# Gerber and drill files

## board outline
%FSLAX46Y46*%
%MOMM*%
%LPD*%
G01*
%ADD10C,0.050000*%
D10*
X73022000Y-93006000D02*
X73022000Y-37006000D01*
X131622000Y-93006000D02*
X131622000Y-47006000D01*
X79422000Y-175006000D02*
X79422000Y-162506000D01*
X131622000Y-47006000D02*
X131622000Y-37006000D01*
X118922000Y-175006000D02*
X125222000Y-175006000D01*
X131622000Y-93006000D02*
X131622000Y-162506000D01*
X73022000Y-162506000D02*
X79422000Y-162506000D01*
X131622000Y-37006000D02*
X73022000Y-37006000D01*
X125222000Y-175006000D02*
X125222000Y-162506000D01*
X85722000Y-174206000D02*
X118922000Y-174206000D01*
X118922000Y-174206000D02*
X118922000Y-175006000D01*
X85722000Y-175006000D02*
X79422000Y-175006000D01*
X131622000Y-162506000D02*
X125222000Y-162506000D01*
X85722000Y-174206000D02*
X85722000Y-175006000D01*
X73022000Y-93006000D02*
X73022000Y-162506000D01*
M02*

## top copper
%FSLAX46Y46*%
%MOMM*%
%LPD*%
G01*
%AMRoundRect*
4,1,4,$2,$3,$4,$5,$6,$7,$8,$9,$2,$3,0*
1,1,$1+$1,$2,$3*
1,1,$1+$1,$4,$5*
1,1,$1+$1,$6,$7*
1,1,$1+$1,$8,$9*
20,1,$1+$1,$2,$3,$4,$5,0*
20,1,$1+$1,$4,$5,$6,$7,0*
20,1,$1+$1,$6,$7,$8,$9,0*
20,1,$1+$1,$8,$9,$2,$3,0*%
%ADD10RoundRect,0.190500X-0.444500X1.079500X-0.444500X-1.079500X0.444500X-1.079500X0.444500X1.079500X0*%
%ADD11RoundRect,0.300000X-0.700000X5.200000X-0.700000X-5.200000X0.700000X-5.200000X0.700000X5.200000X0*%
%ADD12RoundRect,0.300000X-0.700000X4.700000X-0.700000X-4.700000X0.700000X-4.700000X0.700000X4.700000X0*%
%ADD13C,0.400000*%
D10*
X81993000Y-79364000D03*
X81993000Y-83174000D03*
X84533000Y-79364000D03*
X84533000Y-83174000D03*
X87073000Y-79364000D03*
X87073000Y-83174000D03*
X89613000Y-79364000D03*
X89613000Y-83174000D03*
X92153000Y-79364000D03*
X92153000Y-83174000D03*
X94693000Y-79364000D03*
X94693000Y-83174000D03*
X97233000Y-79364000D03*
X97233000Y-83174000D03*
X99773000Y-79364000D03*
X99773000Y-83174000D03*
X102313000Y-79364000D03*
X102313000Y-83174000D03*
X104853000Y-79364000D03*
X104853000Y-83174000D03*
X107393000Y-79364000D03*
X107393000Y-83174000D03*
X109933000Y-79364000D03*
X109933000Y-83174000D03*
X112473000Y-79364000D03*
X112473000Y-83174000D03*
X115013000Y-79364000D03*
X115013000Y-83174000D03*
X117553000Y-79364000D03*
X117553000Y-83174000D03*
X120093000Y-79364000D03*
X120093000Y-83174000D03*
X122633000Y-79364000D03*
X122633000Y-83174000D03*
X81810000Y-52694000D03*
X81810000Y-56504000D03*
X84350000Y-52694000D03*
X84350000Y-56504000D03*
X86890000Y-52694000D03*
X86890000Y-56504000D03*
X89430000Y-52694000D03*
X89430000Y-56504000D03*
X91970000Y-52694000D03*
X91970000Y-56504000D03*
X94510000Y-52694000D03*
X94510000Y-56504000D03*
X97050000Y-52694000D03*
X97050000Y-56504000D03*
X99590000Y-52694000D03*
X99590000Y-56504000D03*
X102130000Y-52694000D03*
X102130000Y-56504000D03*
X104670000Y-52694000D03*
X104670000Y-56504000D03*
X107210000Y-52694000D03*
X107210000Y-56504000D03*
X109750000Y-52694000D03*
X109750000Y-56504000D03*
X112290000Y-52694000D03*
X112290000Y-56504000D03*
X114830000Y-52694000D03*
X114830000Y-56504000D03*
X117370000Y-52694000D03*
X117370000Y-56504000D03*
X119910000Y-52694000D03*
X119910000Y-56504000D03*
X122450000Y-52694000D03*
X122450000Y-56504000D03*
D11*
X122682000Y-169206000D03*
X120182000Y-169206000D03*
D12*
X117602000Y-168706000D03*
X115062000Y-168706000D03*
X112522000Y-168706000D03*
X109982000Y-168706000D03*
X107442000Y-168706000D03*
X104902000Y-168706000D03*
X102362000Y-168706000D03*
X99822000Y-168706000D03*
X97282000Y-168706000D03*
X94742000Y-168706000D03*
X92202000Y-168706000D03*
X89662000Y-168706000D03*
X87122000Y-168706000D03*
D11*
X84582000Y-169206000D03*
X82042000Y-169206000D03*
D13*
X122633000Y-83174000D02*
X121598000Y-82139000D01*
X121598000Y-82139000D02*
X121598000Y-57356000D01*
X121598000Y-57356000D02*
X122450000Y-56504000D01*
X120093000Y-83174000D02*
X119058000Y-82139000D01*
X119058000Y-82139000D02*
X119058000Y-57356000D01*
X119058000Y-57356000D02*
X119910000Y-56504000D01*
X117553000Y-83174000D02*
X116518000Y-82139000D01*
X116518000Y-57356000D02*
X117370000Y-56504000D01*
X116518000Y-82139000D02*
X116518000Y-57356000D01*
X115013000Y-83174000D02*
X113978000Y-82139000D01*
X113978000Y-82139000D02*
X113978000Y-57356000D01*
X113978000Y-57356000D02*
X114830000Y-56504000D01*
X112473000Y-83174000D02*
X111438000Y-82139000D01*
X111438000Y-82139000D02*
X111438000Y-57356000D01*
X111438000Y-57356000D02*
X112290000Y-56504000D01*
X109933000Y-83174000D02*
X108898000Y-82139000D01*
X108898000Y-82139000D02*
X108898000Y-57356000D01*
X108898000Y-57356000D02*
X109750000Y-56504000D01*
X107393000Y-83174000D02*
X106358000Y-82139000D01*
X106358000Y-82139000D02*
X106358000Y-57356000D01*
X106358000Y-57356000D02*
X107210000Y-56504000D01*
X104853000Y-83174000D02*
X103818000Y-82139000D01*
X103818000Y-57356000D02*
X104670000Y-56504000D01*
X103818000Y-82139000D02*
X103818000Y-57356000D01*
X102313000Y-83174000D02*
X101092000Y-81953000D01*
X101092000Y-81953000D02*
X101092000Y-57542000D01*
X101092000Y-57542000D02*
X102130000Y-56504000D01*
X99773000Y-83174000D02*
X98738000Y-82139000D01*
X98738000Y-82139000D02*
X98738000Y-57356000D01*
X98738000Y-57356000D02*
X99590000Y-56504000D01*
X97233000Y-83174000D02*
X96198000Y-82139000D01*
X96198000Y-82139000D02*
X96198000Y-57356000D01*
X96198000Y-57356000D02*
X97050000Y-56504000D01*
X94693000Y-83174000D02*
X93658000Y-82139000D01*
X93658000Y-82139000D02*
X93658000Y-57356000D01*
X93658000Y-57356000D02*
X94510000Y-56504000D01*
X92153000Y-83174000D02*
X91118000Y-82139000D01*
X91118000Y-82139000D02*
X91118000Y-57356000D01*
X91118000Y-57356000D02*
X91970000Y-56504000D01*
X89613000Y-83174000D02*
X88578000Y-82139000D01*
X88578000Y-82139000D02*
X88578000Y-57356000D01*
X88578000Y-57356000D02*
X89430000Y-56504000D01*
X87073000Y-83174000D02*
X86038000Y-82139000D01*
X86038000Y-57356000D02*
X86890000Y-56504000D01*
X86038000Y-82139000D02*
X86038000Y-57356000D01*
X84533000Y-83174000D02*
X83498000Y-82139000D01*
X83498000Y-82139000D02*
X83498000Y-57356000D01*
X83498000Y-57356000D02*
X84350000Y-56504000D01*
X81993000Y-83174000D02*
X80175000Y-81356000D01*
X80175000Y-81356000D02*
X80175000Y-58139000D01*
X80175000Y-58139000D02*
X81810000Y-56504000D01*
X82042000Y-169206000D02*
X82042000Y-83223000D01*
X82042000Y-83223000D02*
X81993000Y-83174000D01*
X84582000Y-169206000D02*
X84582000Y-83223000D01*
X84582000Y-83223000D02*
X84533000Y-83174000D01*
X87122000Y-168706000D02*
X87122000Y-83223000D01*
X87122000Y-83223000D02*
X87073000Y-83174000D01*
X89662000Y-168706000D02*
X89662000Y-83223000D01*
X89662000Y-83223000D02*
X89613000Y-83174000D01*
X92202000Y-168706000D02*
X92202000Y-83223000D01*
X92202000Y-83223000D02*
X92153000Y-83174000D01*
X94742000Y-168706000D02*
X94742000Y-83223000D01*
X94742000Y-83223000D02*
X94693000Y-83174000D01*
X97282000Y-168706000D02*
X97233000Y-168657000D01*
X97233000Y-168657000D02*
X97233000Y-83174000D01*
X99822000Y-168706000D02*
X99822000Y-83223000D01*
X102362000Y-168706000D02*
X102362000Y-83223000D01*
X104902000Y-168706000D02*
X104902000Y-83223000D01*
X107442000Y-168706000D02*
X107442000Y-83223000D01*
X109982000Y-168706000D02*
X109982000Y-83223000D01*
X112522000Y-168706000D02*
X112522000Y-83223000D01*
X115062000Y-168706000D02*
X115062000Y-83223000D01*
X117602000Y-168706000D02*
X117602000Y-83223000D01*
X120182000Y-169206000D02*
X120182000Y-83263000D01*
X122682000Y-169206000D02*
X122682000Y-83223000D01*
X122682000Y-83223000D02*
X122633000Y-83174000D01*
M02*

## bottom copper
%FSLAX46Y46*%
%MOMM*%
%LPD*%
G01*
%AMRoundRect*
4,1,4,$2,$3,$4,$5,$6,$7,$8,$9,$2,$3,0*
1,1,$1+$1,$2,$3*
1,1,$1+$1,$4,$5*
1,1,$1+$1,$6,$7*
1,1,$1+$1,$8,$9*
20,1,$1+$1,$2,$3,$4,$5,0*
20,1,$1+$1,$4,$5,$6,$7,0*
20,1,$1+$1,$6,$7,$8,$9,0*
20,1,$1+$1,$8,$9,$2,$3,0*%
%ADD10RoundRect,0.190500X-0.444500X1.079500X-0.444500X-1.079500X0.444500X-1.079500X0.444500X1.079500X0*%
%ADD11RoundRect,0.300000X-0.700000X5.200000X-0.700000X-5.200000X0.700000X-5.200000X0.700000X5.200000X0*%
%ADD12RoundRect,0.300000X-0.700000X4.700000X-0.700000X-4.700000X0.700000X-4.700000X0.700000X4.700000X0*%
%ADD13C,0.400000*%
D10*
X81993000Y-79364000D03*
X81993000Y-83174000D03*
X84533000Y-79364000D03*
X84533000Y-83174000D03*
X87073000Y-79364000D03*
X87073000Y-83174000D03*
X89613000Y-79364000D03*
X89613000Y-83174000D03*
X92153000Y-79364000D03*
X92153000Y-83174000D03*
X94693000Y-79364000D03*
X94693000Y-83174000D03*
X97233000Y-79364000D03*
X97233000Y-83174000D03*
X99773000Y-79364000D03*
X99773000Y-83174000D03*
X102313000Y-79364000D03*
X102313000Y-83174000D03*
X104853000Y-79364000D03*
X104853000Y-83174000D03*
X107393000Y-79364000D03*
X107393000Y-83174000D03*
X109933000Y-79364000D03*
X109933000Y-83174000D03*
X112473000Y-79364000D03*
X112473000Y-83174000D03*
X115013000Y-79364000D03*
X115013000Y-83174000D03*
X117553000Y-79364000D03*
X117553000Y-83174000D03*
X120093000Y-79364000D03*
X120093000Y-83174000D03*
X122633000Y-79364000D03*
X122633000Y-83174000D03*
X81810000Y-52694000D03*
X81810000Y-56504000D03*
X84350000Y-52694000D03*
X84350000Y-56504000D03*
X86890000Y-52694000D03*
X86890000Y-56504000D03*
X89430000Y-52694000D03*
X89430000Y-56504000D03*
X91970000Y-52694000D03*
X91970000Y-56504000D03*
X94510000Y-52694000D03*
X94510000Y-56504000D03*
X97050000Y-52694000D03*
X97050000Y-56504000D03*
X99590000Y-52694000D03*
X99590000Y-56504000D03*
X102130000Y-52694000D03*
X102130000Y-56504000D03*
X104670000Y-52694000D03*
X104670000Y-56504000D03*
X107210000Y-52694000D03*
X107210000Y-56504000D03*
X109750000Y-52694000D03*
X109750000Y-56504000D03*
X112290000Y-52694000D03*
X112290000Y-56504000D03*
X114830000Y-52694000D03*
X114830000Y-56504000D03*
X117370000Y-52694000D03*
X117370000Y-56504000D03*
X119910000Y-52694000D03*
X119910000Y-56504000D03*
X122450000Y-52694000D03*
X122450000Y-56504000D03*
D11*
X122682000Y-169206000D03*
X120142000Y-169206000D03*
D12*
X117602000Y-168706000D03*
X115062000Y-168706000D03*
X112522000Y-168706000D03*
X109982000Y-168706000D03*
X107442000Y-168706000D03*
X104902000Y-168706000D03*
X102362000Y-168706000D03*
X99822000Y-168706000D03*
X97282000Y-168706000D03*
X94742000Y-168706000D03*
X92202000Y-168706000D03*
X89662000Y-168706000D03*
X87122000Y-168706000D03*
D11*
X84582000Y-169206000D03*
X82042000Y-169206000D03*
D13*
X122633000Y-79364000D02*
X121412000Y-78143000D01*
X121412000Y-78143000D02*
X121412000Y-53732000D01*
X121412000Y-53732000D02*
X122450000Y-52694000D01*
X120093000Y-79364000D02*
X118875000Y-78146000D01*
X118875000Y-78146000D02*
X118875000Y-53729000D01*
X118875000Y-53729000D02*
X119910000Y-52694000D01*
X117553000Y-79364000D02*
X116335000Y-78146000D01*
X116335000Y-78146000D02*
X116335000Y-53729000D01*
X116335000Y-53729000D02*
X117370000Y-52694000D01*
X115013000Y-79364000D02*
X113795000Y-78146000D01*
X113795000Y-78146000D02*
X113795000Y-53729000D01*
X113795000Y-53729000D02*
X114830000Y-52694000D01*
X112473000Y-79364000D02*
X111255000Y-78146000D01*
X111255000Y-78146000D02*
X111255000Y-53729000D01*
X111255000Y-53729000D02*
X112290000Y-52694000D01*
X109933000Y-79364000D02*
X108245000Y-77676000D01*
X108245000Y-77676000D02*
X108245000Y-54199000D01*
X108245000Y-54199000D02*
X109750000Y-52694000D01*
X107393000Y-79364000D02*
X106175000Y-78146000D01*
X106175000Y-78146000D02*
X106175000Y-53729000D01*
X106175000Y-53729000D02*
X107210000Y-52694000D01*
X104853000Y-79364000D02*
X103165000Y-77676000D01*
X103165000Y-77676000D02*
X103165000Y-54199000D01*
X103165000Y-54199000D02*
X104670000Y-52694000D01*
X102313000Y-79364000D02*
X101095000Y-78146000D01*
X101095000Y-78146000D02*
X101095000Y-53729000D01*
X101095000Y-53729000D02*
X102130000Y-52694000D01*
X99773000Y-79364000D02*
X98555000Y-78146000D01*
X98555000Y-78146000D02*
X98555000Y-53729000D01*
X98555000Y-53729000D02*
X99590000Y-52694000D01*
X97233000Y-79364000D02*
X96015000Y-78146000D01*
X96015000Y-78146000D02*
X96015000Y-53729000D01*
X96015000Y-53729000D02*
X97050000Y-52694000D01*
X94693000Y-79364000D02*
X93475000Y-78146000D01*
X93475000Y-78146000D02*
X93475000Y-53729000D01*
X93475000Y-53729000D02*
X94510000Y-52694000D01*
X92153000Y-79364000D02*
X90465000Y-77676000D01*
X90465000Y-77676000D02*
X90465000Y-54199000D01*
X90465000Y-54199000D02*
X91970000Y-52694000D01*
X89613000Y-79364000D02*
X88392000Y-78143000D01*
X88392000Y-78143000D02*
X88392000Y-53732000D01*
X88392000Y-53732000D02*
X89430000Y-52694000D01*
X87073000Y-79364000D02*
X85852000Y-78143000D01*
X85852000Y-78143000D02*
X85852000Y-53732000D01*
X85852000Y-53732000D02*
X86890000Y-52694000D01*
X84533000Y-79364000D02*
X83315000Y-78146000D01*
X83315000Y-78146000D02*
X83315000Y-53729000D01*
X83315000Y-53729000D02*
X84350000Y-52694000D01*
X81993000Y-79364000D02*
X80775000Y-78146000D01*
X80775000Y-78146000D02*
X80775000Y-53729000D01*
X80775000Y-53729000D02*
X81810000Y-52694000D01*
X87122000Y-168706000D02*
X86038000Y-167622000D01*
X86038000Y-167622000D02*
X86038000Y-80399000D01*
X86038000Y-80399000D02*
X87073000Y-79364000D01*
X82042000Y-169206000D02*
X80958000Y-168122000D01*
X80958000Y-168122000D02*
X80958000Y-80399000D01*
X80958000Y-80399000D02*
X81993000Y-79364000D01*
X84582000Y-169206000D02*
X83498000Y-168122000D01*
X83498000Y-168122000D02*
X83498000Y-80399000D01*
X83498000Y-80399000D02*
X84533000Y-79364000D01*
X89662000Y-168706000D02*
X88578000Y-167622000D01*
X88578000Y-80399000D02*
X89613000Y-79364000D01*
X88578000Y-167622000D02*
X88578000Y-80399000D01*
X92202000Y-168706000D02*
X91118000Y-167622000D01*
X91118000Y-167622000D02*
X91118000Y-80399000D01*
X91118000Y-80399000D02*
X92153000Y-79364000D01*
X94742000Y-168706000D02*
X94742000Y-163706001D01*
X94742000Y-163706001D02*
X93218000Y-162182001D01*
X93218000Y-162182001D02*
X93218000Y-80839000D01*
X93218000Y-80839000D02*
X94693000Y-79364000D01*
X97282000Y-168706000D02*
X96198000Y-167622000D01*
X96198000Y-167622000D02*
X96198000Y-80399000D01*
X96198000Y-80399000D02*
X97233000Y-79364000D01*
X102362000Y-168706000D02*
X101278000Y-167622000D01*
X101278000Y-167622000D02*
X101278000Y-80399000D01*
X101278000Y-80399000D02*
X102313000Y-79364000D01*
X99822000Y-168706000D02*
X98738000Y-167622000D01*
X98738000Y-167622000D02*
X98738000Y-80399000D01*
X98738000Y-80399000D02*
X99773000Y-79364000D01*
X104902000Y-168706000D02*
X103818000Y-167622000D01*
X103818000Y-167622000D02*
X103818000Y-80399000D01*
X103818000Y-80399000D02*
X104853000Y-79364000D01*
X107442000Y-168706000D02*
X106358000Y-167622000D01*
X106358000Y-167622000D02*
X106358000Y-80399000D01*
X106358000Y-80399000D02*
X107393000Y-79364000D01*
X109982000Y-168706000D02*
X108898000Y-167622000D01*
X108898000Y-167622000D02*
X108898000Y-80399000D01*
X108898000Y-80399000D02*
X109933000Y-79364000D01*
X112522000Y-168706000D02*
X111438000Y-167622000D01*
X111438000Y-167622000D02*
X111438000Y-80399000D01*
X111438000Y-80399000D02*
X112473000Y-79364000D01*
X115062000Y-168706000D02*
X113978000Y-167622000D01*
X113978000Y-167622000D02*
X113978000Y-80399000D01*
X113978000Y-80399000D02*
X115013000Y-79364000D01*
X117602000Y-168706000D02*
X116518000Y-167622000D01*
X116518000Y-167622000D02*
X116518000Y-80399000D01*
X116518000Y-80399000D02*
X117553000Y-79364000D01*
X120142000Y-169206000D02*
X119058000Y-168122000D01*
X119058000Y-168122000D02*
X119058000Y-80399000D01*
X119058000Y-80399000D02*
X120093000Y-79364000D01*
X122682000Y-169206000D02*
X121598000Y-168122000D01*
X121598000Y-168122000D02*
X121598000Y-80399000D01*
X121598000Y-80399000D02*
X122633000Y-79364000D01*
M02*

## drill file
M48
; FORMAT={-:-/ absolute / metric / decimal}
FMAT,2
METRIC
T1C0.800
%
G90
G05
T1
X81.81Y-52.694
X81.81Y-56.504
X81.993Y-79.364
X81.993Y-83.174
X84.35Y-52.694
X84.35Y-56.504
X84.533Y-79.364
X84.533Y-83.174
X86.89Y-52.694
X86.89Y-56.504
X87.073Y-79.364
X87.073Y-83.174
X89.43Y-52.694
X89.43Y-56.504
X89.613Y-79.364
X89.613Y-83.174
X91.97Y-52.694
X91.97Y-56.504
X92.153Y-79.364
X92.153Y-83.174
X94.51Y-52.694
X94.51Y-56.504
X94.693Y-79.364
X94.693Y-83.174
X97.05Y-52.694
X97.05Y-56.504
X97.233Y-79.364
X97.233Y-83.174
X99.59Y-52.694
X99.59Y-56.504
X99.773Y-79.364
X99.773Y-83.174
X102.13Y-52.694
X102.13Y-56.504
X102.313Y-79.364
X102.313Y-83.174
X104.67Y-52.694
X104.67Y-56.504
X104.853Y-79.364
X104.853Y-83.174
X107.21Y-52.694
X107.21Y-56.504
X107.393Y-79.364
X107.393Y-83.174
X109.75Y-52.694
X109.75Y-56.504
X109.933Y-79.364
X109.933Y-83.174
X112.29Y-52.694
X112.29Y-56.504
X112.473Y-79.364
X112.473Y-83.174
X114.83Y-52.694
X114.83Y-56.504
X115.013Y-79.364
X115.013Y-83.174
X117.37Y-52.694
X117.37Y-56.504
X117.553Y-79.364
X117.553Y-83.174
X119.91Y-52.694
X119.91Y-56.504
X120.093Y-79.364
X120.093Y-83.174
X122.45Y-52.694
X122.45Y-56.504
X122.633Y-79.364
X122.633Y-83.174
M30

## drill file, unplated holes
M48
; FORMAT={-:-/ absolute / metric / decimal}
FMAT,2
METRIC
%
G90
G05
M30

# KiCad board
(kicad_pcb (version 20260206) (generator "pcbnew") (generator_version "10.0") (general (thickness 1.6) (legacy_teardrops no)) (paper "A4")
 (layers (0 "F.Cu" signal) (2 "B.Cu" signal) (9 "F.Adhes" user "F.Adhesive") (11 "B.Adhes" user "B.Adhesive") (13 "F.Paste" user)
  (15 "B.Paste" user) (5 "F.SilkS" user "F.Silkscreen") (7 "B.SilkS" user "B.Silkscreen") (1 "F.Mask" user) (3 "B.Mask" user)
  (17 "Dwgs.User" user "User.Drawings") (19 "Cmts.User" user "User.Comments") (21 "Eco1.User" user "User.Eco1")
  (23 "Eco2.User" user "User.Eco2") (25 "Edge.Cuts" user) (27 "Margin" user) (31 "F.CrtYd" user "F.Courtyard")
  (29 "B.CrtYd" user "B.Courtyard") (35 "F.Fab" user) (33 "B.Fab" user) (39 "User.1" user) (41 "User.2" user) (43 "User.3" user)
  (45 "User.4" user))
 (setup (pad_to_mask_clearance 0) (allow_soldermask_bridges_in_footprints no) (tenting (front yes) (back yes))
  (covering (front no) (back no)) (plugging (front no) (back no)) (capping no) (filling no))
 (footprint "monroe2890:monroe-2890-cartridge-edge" (layer "F.Cu") (at 122.682 168.706 -90)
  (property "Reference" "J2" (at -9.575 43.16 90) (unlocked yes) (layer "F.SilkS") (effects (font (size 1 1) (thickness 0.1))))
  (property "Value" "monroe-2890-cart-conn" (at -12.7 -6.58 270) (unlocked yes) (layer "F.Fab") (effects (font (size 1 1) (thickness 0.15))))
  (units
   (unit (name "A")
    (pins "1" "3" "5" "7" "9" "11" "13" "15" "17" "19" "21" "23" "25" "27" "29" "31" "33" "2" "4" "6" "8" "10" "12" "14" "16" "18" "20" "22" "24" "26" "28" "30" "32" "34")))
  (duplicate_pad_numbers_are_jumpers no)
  (pad "1" smd roundrect (at 0.5 0 270) (size 11 2) (layers "F.Cu" "F.Mask" "F.Paste") (roundrect_rratio 0.15) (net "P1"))
  (pad "2" connect roundrect (at 0.5 0 270) (size 11 2) (layers "B.Cu" "B.Mask") (roundrect_rratio 0.15) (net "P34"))
  (pad "3" smd roundrect (at 0.5 2.5 270) (size 11 2) (layers "F.Cu" "F.Mask" "F.Paste") (roundrect_rratio 0.15) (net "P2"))
  (pad "4" connect roundrect (at 0.5 2.54 270) (size 11 2) (layers "B.Cu" "B.Mask") (roundrect_rratio 0.15) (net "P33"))
  (pad "5" smd roundrect (at 0 5.08 270) (size 10 2) (layers "F.Cu" "F.Mask" "F.Paste") (roundrect_rratio 0.15) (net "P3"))
  (pad "6" connect roundrect (at 0 5.08 270) (size 10 2) (layers "B.Cu" "B.Mask") (roundrect_rratio 0.15) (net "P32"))
  (pad "7" smd roundrect (at 0 7.62 270) (size 10 2) (layers "F.Cu" "F.Mask" "F.Paste") (roundrect_rratio 0.15) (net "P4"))
  (pad "8" connect roundrect (at 0 7.62 270) (size 10 2) (layers "B.Cu" "B.Mask") (roundrect_rratio 0.15) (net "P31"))
  (pad "9" smd roundrect (at 0 10.16 270) (size 10 2) (layers "F.Cu" "F.Mask" "F.Paste") (roundrect_rratio 0.15) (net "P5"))
  (pad "10" connect roundrect (at 0 10.16 270) (size 10 2) (layers "B.Cu" "B.Mask") (roundrect_rratio 0.15) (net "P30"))
  (pad "11" smd roundrect (at 0 12.7 270) (size 10 2) (layers "F.Cu" "F.Mask" "F.Paste") (roundrect_rratio 0.15) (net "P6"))
  (pad "12" connect roundrect (at 0 12.7 270) (size 10 2) (layers "B.Cu" "B.Mask") (roundrect_rratio 0.15) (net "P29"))
  (pad "13" smd roundrect (at 0 15.24 270) (size 10 2) (layers "F.Cu" "F.Mask" "F.Paste") (roundrect_rratio 0.15) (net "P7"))
  (pad "14" connect roundrect (at 0 15.24 270) (size 10 2) (layers "B.Cu" "B.Mask") (roundrect_rratio 0.15) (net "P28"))
  (pad "15" smd roundrect (at 0 17.78 270) (size 10 2) (layers "F.Cu" "F.Mask" "F.Paste") (roundrect_rratio 0.15) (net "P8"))
  (pad "16" connect roundrect (at 0 17.78 270) (size 10 2) (layers "B.Cu" "B.Mask") (roundrect_rratio 0.15) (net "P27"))
  (pad "17" smd roundrect (at 0 20.32 270) (size 10 2) (layers "F.Cu" "F.Mask" "F.Paste") (roundrect_rratio 0.15) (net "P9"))
  (pad "18" connect roundrect (at 0 20.32 270) (size 10 2) (layers "B.Cu" "B.Mask") (roundrect_rratio 0.15) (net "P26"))
  (pad "19" smd roundrect (at 0 22.86 270) (size 10 2) (layers "F.Cu" "F.Mask" "F.Paste") (roundrect_rratio 0.15) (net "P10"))
  (pad "20" connect roundrect (at 0 22.86 270) (size 10 2) (layers "B.Cu" "B.Mask") (roundrect_rratio 0.15) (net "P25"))
  (pad "21" smd roundrect (at 0 25.4 270) (size 10 2) (layers "F.Cu" "F.Mask" "F.Paste") (roundrect_rratio 0.15) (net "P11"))
  (pad "22" connect roundrect (at 0 25.4 270) (size 10 2) (layers "B.Cu" "B.Mask") (roundrect_rratio 0.15) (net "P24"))
  (pad "23" smd roundrect (at 0 27.94 270) (size 10 2) (layers "F.Cu" "F.Mask" "F.Paste") (roundrect_rratio 0.15) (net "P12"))
  (pad "24" connect roundrect (at 0 27.94 270) (size 10 2) (layers "B.Cu" "B.Mask") (roundrect_rratio 0.15) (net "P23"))
  (pad "25" smd roundrect (at 0 30.48 270) (size 10 2) (layers "F.Cu" "F.Mask" "F.Paste") (roundrect_rratio 0.15) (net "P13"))
  (pad "26" connect roundrect (at 0 30.48 270) (size 10 2) (layers "B.Cu" "B.Mask") (roundrect_rratio 0.15) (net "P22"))
  (pad "27" smd roundrect (at 0 33.02 270) (size 10 2) (layers "F.Cu" "F.Mask" "F.Paste") (roundrect_rratio 0.15) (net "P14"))
  (pad "28" connect roundrect (at 0 33.02 270) (size 10 2) (layers "B.Cu" "B.Mask") (roundrect_rratio 0.15) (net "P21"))
  (pad "29" smd roundrect (at 0 35.56 270) (size 10 2) (layers "F.Cu" "F.Mask" "F.Paste") (roundrect_rratio 0.15) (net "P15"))
  (pad "30" connect roundrect (at 0 35.56 270) (size 10 2) (layers "B.Cu" "B.Mask") (roundrect_rratio 0.15) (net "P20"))
  (pad "31" smd roundrect (at 0.5 38.1 270) (size 11 2) (layers "F.Cu" "F.Mask" "F.Paste") (roundrect_rratio 0.15) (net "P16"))
  (pad "32" connect roundrect (at 0.5 38.1 270) (size 11 2) (layers "B.Cu" "B.Mask") (roundrect_rratio 0.15) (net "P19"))
  (pad "33" smd roundrect (at 0.5 40.64 270) (size 11 2) (layers "F.Cu" "F.Mask" "F.Paste") (roundrect_rratio 0.15) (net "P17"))
  (pad "34" connect roundrect (at 0.5 40.64 270) (size 11 2) (layers "B.Cu" "B.Mask") (roundrect_rratio 0.15) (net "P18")))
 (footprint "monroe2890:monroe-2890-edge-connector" (layer "F.Cu") (at 111.457 78.856 -90)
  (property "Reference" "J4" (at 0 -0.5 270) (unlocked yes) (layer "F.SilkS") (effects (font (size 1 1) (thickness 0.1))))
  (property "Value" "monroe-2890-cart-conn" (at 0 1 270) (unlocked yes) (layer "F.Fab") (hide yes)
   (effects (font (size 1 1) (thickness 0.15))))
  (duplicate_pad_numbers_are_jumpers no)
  (pad "1" thru_hole roundrect (at 4.318 -11.176 270) (size 2.54 1.27) (drill 0.8) (layers "*.Cu" "*.Mask") (remove_unused_layers no)
   (roundrect_rratio 0.15) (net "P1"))
  (pad "2" thru_hole roundrect (at 0.508 -11.176 270) (size 2.54 1.27) (drill 0.8) (layers "*.Cu" "*.Mask") (remove_unused_layers no)
   (roundrect_rratio 0.15) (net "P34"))
  (pad "3" thru_hole roundrect (at 4.318 -8.636 270) (size 2.54 1.27) (drill 0.8) (layers "*.Cu" "*.Mask") (remove_unused_layers no)
   (roundrect_rratio 0.15) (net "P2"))
  (pad "4" thru_hole roundrect (at 0.508 -8.636 270) (size 2.54 1.27) (drill 0.8) (layers "*.Cu" "*.Mask") (remove_unused_layers no)
   (roundrect_rratio 0.15) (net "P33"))
  (pad "5" thru_hole roundrect (at 4.318 -6.096 270) (size 2.54 1.27) (drill 0.8) (layers "*.Cu" "*.Mask") (remove_unused_layers no)
   (roundrect_rratio 0.15) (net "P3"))
  (pad "6" thru_hole roundrect (at 0.508 -6.096 270) (size 2.54 1.27) (drill 0.8) (layers "*.Cu" "*.Mask") (remove_unused_layers no)
   (roundrect_rratio 0.15) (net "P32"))
  (pad "7" thru_hole roundrect (at 4.318 -3.556 270) (size 2.54 1.27) (drill 0.8) (layers "*.Cu" "*.Mask") (remove_unused_layers no)
   (roundrect_rratio 0.15) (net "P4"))
  (pad "8" thru_hole roundrect (at 0.508 -3.556 270) (size 2.54 1.27) (drill 0.8) (layers "*.Cu" "*.Mask") (remove_unused_layers no)
   (roundrect_rratio 0.15) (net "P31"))
  (pad "9" thru_hole roundrect (at 4.318 -1.016 270) (size 2.54 1.27) (drill 0.8) (layers "*.Cu" "*.Mask") (remove_unused_layers no)
   (roundrect_rratio 0.15) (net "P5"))
  (pad "10" thru_hole roundrect (at 0.508 -1.016 270) (size 2.54 1.27) (drill 0.8) (layers "*.Cu" "*.Mask") (remove_unused_layers no)
   (roundrect_rratio 0.15) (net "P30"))
  (pad "11" thru_hole roundrect (at 4.318 1.524 270) (size 2.54 1.27) (drill 0.8) (layers "*.Cu" "*.Mask") (remove_unused_layers no)
   (roundrect_rratio 0.15) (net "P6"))
  (pad "12" thru_hole roundrect (at 0.508 1.524 270) (size 2.54 1.27) (drill 0.8) (layers "*.Cu" "*.Mask") (remove_unused_layers no)
   (roundrect_rratio 0.15) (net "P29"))
  (pad "13" thru_hole roundrect (at 4.318 4.064 270) (size 2.54 1.27) (drill 0.8) (layers "*.Cu" "*.Mask") (remove_unused_layers no)
   (roundrect_rratio 0.15) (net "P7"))
  (pad "14" thru_hole roundrect (at 0.508 4.064 270) (size 2.54 1.27) (drill 0.8) (layers "*.Cu" "*.Mask") (remove_unused_layers no)
   (roundrect_rratio 0.15) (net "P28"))
  (pad "15" thru_hole roundrect (at 4.318 6.604 270) (size 2.54 1.27) (drill 0.8) (layers "*.Cu" "*.Mask") (remove_unused_layers no)
   (roundrect_rratio 0.15) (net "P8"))
  (pad "16" thru_hole roundrect (at 0.508 6.604 270) (size 2.54 1.27) (drill 0.8) (layers "*.Cu" "*.Mask") (remove_unused_layers no)
   (roundrect_rratio 0.15) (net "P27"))
  (pad "17" thru_hole roundrect (at 4.318 9.144 270) (size 2.54 1.27) (drill 0.8) (layers "*.Cu" "*.Mask") (remove_unused_layers no)
   (roundrect_rratio 0.15) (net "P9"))
  (pad "18" thru_hole roundrect (at 0.508 9.144 270) (size 2.54 1.27) (drill 0.8) (layers "*.Cu" "*.Mask") (remove_unused_layers no)
   (roundrect_rratio 0.15) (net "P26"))
  (pad "19" thru_hole roundrect (at 4.318 11.684 270) (size 2.54 1.27) (drill 0.8) (layers "*.Cu" "*.Mask") (remove_unused_layers no)
   (roundrect_rratio 0.15) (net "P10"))
  (pad "20" thru_hole roundrect (at 0.508 11.684 270) (size 2.54 1.27) (drill 0.8) (layers "*.Cu" "*.Mask") (remove_unused_layers no)
   (roundrect_rratio 0.15) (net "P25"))
  (pad "21" thru_hole roundrect (at 4.318 14.224 270) (size 2.54 1.27) (drill 0.8) (layers "*.Cu" "*.Mask") (remove_unused_layers no)
   (roundrect_rratio 0.15) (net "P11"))
  (pad "22" thru_hole roundrect (at 0.508 14.224 270) (size 2.54 1.27) (drill 0.8) (layers "*.Cu" "*.Mask") (remove_unused_layers no)
   (roundrect_rratio 0.15) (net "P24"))
  (pad "23" thru_hole roundrect (at 4.318 16.764 270) (size 2.54 1.27) (drill 0.8) (layers "*.Cu" "*.Mask") (remove_unused_layers no)
   (roundrect_rratio 0.15) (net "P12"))
  (pad "24" thru_hole roundrect (at 0.508 16.764 270) (size 2.54 1.27) (drill 0.8) (layers "*.Cu" "*.Mask") (remove_unused_layers no)
   (roundrect_rratio 0.15) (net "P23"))
  (pad "25" thru_hole roundrect (at 4.318 19.304 270) (size 2.54 1.27) (drill 0.8) (layers "*.Cu" "*.Mask") (remove_unused_layers no)
   (roundrect_rratio 0.15) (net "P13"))
  (pad "26" thru_hole roundrect (at 0.508 19.304 270) (size 2.54 1.27) (drill 0.8) (layers "*.Cu" "*.Mask") (remove_unused_layers no)
   (roundrect_rratio 0.15) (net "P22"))
  (pad "27" thru_hole roundrect (at 4.318 21.844 270) (size 2.54 1.27) (drill 0.8) (layers "*.Cu" "*.Mask") (remove_unused_layers no)
   (roundrect_rratio 0.15) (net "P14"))
  (pad "28" thru_hole roundrect (at 0.508 21.844 270) (size 2.54 1.27) (drill 0.8) (layers "*.Cu" "*.Mask") (remove_unused_layers no)
   (roundrect_rratio 0.15) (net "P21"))
  (pad "29" thru_hole roundrect (at 4.318 24.384 270) (size 2.54 1.27) (drill 0.8) (layers "*.Cu" "*.Mask") (remove_unused_layers no)
   (roundrect_rratio 0.15) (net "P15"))
  (pad "30" thru_hole roundrect (at 0.508 24.384 270) (size 2.54 1.27) (drill 0.8) (layers "*.Cu" "*.Mask") (remove_unused_layers no)
   (roundrect_rratio 0.15) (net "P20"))
  (pad "31" thru_hole roundrect (at 4.318 26.924 270) (size 2.54 1.27) (drill 0.8) (layers "*.Cu" "*.Mask") (remove_unused_layers no)
   (roundrect_rratio 0.15) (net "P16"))
  (pad "32" thru_hole roundrect (at 0.508 26.924 270) (size 2.54 1.27) (drill 0.8) (layers "*.Cu" "*.Mask") (remove_unused_layers no)
   (roundrect_rratio 0.15) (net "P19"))
  (pad "33" thru_hole roundrect (at 4.318 29.464 270) (size 2.54 1.27) (drill 0.8) (layers "*.Cu" "*.Mask") (remove_unused_layers no)
   (roundrect_rratio 0.15) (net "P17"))
  (pad "34" thru_hole roundrect (at 0.508 29.464 270) (size 2.54 1.27) (drill 0.8) (layers "*.Cu" "*.Mask") (remove_unused_layers no)
   (roundrect_rratio 0.15) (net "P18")))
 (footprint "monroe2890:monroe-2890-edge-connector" (layer "F.Cu") (at 111.274 52.186 -90)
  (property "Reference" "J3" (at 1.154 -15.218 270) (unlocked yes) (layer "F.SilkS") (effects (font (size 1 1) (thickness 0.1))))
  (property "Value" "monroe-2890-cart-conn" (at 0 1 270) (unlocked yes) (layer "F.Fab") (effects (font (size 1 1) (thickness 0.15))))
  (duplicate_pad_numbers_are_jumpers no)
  (pad "1" thru_hole roundrect (at 4.318 -11.176 270) (size 2.54 1.27) (drill 0.8) (layers "*.Cu" "*.Mask") (remove_unused_layers no)
   (roundrect_rratio 0.15) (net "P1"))
  (pad "2" thru_hole roundrect (at 0.508 -11.176 270) (size 2.54 1.27) (drill 0.8) (layers "*.Cu" "*.Mask") (remove_unused_layers no)
   (roundrect_rratio 0.15) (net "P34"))
  (pad "3" thru_hole roundrect (at 4.318 -8.636 270) (size 2.54 1.27) (drill 0.8) (layers "*.Cu" "*.Mask") (remove_unused_layers no)
   (roundrect_rratio 0.15) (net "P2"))
  (pad "4" thru_hole roundrect (at 0.508 -8.636 270) (size 2.54 1.27) (drill 0.8) (layers "*.Cu" "*.Mask") (remove_unused_layers no)
   (roundrect_rratio 0.15) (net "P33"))
  (pad "5" thru_hole roundrect (at 4.318 -6.096 270) (size 2.54 1.27) (drill 0.8) (layers "*.Cu" "*.Mask") (remove_unused_layers no)
   (roundrect_rratio 0.15) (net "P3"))
  (pad "6" thru_hole roundrect (at 0.508 -6.096 270) (size 2.54 1.27) (drill 0.8) (layers "*.Cu" "*.Mask") (remove_unused_layers no)
   (roundrect_rratio 0.15) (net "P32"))
  (pad "7" thru_hole roundrect (at 4.318 -3.556 270) (size 2.54 1.27) (drill 0.8) (layers "*.Cu" "*.Mask") (remove_unused_layers no)
   (roundrect_rratio 0.15) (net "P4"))
  (pad "8" thru_hole roundrect (at 0.508 -3.556 270) (size 2.54 1.27) (drill 0.8) (layers "*.Cu" "*.Mask") (remove_unused_layers no)
   (roundrect_rratio 0.15) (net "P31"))
  (pad "9" thru_hole roundrect (at 4.318 -1.016 270) (size 2.54 1.27) (drill 0.8) (layers "*.Cu" "*.Mask") (remove_unused_layers no)
   (roundrect_rratio 0.15) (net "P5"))
  (pad "10" thru_hole roundrect (at 0.508 -1.016 270) (size 2.54 1.27) (drill 0.8) (layers "*.Cu" "*.Mask") (remove_unused_layers no)
   (roundrect_rratio 0.15) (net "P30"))
  (pad "11" thru_hole roundrect (at 4.318 1.524 270) (size 2.54 1.27) (drill 0.8) (layers "*.Cu" "*.Mask") (remove_unused_layers no)
   (roundrect_rratio 0.15) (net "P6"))
  (pad "12" thru_hole roundrect (at 0.508 1.524 270) (size 2.54 1.27) (drill 0.8) (layers "*.Cu" "*.Mask") (remove_unused_layers no)
   (roundrect_rratio 0.15) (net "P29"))
  (pad "13" thru_hole roundrect (at 4.318 4.064 270) (size 2.54 1.27) (drill 0.8) (layers "*.Cu" "*.Mask") (remove_unused_layers no)
   (roundrect_rratio 0.15) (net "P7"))
  (pad "14" thru_hole roundrect (at 0.508 4.064 270) (size 2.54 1.27) (drill 0.8) (layers "*.Cu" "*.Mask") (remove_unused_layers no)
   (roundrect_rratio 0.15) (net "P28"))
  (pad "15" thru_hole roundrect (at 4.318 6.604 270) (size 2.54 1.27) (drill 0.8) (layers "*.Cu" "*.Mask") (remove_unused_layers no)
   (roundrect_rratio 0.15) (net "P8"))
  (pad "16" thru_hole roundrect (at 0.508 6.604 270) (size 2.54 1.27) (drill 0.8) (layers "*.Cu" "*.Mask") (remove_unused_layers no)
   (roundrect_rratio 0.15) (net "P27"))
  (pad "17" thru_hole roundrect (at 4.318 9.144 270) (size 2.54 1.27) (drill 0.8) (layers "*.Cu" "*.Mask") (remove_unused_layers no)
   (roundrect_rratio 0.15) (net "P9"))
  (pad "18" thru_hole roundrect (at 0.508 9.144 270) (size 2.54 1.27) (drill 0.8) (layers "*.Cu" "*.Mask") (remove_unused_layers no)
   (roundrect_rratio 0.15) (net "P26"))
  (pad "19" thru_hole roundrect (at 4.318 11.684 270) (size 2.54 1.27) (drill 0.8) (layers "*.Cu" "*.Mask") (remove_unused_layers no)
   (roundrect_rratio 0.15) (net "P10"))
  (pad "20" thru_hole roundrect (at 0.508 11.684 270) (size 2.54 1.27) (drill 0.8) (layers "*.Cu" "*.Mask") (remove_unused_layers no)
   (roundrect_rratio 0.15) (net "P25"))
  (pad "21" thru_hole roundrect (at 4.318 14.224 270) (size 2.54 1.27) (drill 0.8) (layers "*.Cu" "*.Mask") (remove_unused_layers no)
   (roundrect_rratio 0.15) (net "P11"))
  (pad "22" thru_hole roundrect (at 0.508 14.224 270) (size 2.54 1.27) (drill 0.8) (layers "*.Cu" "*.Mask") (remove_unused_layers no)
   (roundrect_rratio 0.15) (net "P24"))
  (pad "23" thru_hole roundrect (at 4.318 16.764 270) (size 2.54 1.27) (drill 0.8) (layers "*.Cu" "*.Mask") (remove_unused_layers no)
   (roundrect_rratio 0.15) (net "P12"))
  (pad "24" thru_hole roundrect (at 0.508 16.764 270) (size 2.54 1.27) (drill 0.8) (layers "*.Cu" "*.Mask") (remove_unused_layers no)
   (roundrect_rratio 0.15) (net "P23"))
  (pad "25" thru_hole roundrect (at 4.318 19.304 270) (size 2.54 1.27) (drill 0.8) (layers "*.Cu" "*.Mask") (remove_unused_layers no)
   (roundrect_rratio 0.15) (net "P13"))
  (pad "26" thru_hole roundrect (at 0.508 19.304 270) (size 2.54 1.27) (drill 0.8) (layers "*.Cu" "*.Mask") (remove_unused_layers no)
   (roundrect_rratio 0.15) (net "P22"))
  (pad "27" thru_hole roundrect (at 4.318 21.844 270) (size 2.54 1.27) (drill 0.8) (layers "*.Cu" "*.Mask") (remove_unused_layers no)
   (roundrect_rratio 0.15) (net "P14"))
  (pad "28" thru_hole roundrect (at 0.508 21.844 270) (size 2.54 1.27) (drill 0.8) (layers "*.Cu" "*.Mask") (remove_unused_layers no)
   (roundrect_rratio 0.15) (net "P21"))
  (pad "29" thru_hole roundrect (at 4.318 24.384 270) (size 2.54 1.27) (drill 0.8) (layers "*.Cu" "*.Mask") (remove_unused_layers no)
   (roundrect_rratio 0.15) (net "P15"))
  (pad "30" thru_hole roundrect (at 0.508 24.384 270) (size 2.54 1.27) (drill 0.8) (layers "*.Cu" "*.Mask") (remove_unused_layers no)
   (roundrect_rratio 0.15) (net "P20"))
  (pad "31" thru_hole roundrect (at 4.318 26.924 270) (size 2.54 1.27) (drill 0.8) (layers "*.Cu" "*.Mask") (remove_unused_layers no)
   (roundrect_rratio 0.15) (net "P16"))
  (pad "32" thru_hole roundrect (at 0.508 26.924 270) (size 2.54 1.27) (drill 0.8) (layers "*.Cu" "*.Mask") (remove_unused_layers no)
   (roundrect_rratio 0.15) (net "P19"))
  (pad "33" thru_hole roundrect (at 4.318 29.464 270) (size 2.54 1.27) (drill 0.8) (layers "*.Cu" "*.Mask") (remove_unused_layers no)
   (roundrect_rratio 0.15) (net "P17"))
  (pad "34" thru_hole roundrect (at 0.508 29.464 270) (size 2.54 1.27) (drill 0.8) (layers "*.Cu" "*.Mask") (remove_unused_layers no)
   (roundrect_rratio 0.15) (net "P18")))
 (gr_line (start 73.022 93.006) (end 73.022 37.006) (stroke (width 0.05) (type default)) (layer "Edge.Cuts"))
 (gr_line (start 73.022 93.006) (end 73.022 162.506) (stroke (width 0.05) (type default)) (layer "Edge.Cuts"))
 (gr_line (start 73.022 162.506) (end 79.422 162.506) (stroke (width 0.05) (type default)) (layer "Edge.Cuts"))
 (gr_line (start 79.422 175.006) (end 79.422 162.506) (stroke (width 0.05) (type default)) (layer "Edge.Cuts"))
 (gr_line (start 85.722 174.206) (end 85.722 175.006) (stroke (width 0.05) (type default)) (layer "Edge.Cuts"))
 (gr_line (start 85.722 174.206) (end 118.922 174.206) (stroke (width 0.05) (type default)) (layer "Edge.Cuts"))
 (gr_line (start 85.722 175.006) (end 79.422 175.006) (stroke (width 0.05) (type default)) (layer "Edge.Cuts"))
 (gr_line (start 118.922 174.206) (end 118.922 175.006) (stroke (width 0.05) (type default)) (layer "Edge.Cuts"))
 (gr_line (start 118.922 175.006) (end 125.222 175.006) (stroke (width 0.05) (type default)) (layer "Edge.Cuts"))
 (gr_line (start 125.222 175.006) (end 125.222 162.506) (stroke (width 0.05) (type default)) (layer "Edge.Cuts"))
 (gr_line (start 131.622 37.006) (end 73.022 37.006) (stroke (width 0.05) (type default)) (layer "Edge.Cuts"))
 (gr_line (start 131.622 47.006) (end 131.622 37.006) (stroke (width 0.05) (type default)) (layer "Edge.Cuts"))
 (gr_line (start 131.622 93.006) (end 131.622 47.006) (stroke (width 0.05) (type default)) (layer "Edge.Cuts"))
 (gr_line (start 131.622 93.006) (end 131.622 162.506) (stroke (width 0.05) (type default)) (layer "Edge.Cuts"))
 (gr_line (start 131.622 162.506) (end 125.222 162.506) (stroke (width 0.05) (type default)) (layer "Edge.Cuts"))
 (segment (start 98.738 82.139) (end 98.738 57.356) (width 0.4) (layer "F.Cu") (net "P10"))
 (segment (start 99.773 83.174) (end 98.738 82.139) (width 0.4) (layer "F.Cu") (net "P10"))
 (segment (start 99.822 168.706) (end 99.822 83.223) (width 0.4) (layer "F.Cu") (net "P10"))
 (segment (start 98.738 57.356) (end 99.59 56.504) (width 0.4) (layer "F.Cu") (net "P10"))
 (segment (start 113.978 80.399) (end 115.013 79.364) (width 0.4) (layer "B.Cu") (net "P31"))
 (segment (start 113.978 167.622) (end 113.978 80.399) (width 0.4) (layer "B.Cu") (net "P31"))
 (segment (start 113.795 53.729) (end 114.83 52.694) (width 0.4) (layer "B.Cu") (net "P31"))
 (segment (start 113.795 78.146) (end 113.795 53.729) (width 0.4) (layer "B.Cu") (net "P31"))
 (segment (start 115.062 168.706) (end 113.978 167.622) (width 0.4) (layer "B.Cu") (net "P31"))
 (segment (start 115.013 79.364) (end 113.795 78.146) (width 0.4) (layer "B.Cu") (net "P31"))
 (segment (start 115.062 168.706) (end 115.062 83.223) (width 0.4) (layer "F.Cu") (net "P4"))
 (segment (start 115.013 83.174) (end 113.978 82.139) (width 0.4) (layer "F.Cu") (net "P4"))
 (segment (start 113.978 57.356) (end 114.83 56.504) (width 0.4) (layer "F.Cu") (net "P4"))
 (segment (start 113.978 82.139) (end 113.978 57.356) (width 0.4) (layer "F.Cu") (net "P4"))
 (segment (start 84.582 169.206) (end 83.498 168.122) (width 0.4) (layer "B.Cu") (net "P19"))
 (segment (start 83.315 53.729) (end 84.35 52.694) (width 0.4) (layer "B.Cu") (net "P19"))
 (segment (start 84.533 79.364) (end 83.315 78.146) (width 0.4) (layer "B.Cu") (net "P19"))
 (segment (start 83.315 78.146) (end 83.315 53.729) (width 0.4) (layer "B.Cu") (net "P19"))
 (segment (start 83.498 168.122) (end 83.498 80.399) (width 0.4) (layer "B.Cu") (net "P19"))
 (segment (start 83.498 80.399) (end 84.533 79.364) (width 0.4) (layer "B.Cu") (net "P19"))
 (segment (start 93.218 80.839) (end 94.693 79.364) (width 0.4) (layer "B.Cu") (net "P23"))
 (segment (start 93.218 162.182001) (end 93.218 80.839) (width 0.4) (layer "B.Cu") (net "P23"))
 (segment (start 94.742 163.706001) (end 93.218 162.182001) (width 0.4) (layer "B.Cu") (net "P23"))
 (segment (start 93.475 53.729) (end 94.51 52.694) (width 0.4) (layer "B.Cu") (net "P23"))
 (segment (start 94.742 168.706) (end 94.742 163.706001) (width 0.4) (layer "B.Cu") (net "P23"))
 (segment (start 93.475 78.146) (end 93.475 53.729) (width 0.4) (layer "B.Cu") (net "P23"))
 (segment (start 94.693 79.364) (end 93.475 78.146) (width 0.4) (layer "B.Cu") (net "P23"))
 (segment (start 107.393 83.174) (end 106.358 82.139) (width 0.4) (layer "F.Cu") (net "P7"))
 (segment (start 106.358 57.356) (end 107.21 56.504) (width 0.4) (layer "F.Cu") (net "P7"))
 (segment (start 107.442 168.706) (end 107.442 83.223) (width 0.4) (layer "F.Cu") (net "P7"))
 (segment (start 106.358 82.139) (end 106.358 57.356) (width 0.4) (layer "F.Cu") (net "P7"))
 (segment (start 97.233 83.174) (end 96.198 82.139) (width 0.4) (layer "F.Cu") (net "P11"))
 (segment (start 97.233 168.657) (end 97.233 83.174) (width 0.4) (layer "F.Cu") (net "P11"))
 (segment (start 96.198 57.356) (end 97.05 56.504) (width 0.4) (layer "F.Cu") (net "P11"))
 (segment (start 96.198 82.139) (end 96.198 57.356) (width 0.4) (layer "F.Cu") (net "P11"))
 (segment (start 97.282 168.706) (end 97.233 168.657) (width 0.4) (layer "F.Cu") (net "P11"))
 (segment (start 103.818 80.399) (end 104.853 79.364) (width 0.4) (layer "B.Cu") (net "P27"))
 (segment (start 104.853 79.364) (end 103.165 77.676) (width 0.4) (layer "B.Cu") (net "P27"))
 (segment (start 103.165 77.676) (end 103.165 54.199) (width 0.4) (layer "B.Cu") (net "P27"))
 (segment (start 103.818 167.622) (end 103.818 80.399) (width 0.4) (layer "B.Cu") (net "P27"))
 (segment (start 104.902 168.706) (end 103.818 167.622) (width 0.4) (layer "B.Cu") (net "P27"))
 (segment (start 103.165 54.199) (end 104.67 52.694) (width 0.4) (layer "B.Cu") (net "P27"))
 (segment (start 81.993 83.174) (end 80.175 81.356) (width 0.4) (layer "F.Cu") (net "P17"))
 (segment (start 82.042 83.223) (end 81.993 83.174) (width 0.4) (layer "F.Cu") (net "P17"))
 (segment (start 80.175 81.356) (end 80.175 58.139) (width 0.4) (layer "F.Cu") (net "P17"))
 (segment (start 80.175 58.139) (end 81.81 56.504) (width 0.4) (layer "F.Cu") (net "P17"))
 (segment (start 82.042 169.206) (end 82.042 83.223) (width 0.4) (layer "F.Cu") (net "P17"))
 (segment (start 89.613 79.364) (end 88.392 78.143) (width 0.4) (layer "B.Cu") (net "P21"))
 (segment (start 88.392 53.732) (end 89.43 52.694) (width 0.4) (layer "B.Cu") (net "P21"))
 (segment (start 88.578 80.399) (end 89.613 79.364) (width 0.4) (layer "B.Cu") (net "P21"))
 (segment (start 88.578 167.622) (end 88.578 80.399) (width 0.4) (layer "B.Cu") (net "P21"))
 (segment (start 88.392 78.143) (end 88.392 53.732) (width 0.4) (layer "B.Cu") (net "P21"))
 (segment (start 89.662 168.706) (end 88.578 167.622) (width 0.4) (layer "B.Cu") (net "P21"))
 (segment (start 111.255 53.729) (end 112.29 52.694) (width 0.4) (layer "B.Cu") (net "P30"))
 (segment (start 111.255 78.146) (end 111.255 53.729) (width 0.4) (layer "B.Cu") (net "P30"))
 (segment (start 112.473 79.364) (end 111.255 78.146) (width 0.4) (layer "B.Cu") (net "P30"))
 (segment (start 111.438 80.399) (end 112.473 79.364) (width 0.4) (layer "B.Cu") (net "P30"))
 (segment (start 112.522 168.706) (end 111.438 167.622) (width 0.4) (layer "B.Cu") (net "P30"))
 (segment (start 111.438 167.622) (end 111.438 80.399) (width 0.4) (layer "B.Cu") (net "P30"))
 (segment (start 88.578 82.139) (end 88.578 57.356) (width 0.4) (layer "F.Cu") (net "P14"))
 (segment (start 89.662 83.223) (end 89.613 83.174) (width 0.4) (layer "F.Cu") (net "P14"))
 (segment (start 88.578 57.356) (end 89.43 56.504) (width 0.4) (layer "F.Cu") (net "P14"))
 (segment (start 89.662 168.706) (end 89.662 83.223) (width 0.4) (layer "F.Cu") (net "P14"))
 (segment (start 89.613 83.174) (end 88.578 82.139) (width 0.4) (layer "F.Cu") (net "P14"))
 (segment (start 86.038 57.356) (end 86.89 56.504) (width 0.4) (layer "F.Cu") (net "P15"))
 (segment (start 87.122 83.223) (end 87.073 83.174) (width 0.4) (layer "F.Cu") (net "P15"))
 (segment (start 87.073 83.174) (end 86.038 82.139) (width 0.4) (layer "F.Cu") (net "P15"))
 (segment (start 86.038 82.139) (end 86.038 57.356) (width 0.4) (layer "F.Cu") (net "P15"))
 (segment (start 87.122 168.706) (end 87.122 83.223) (width 0.4) (layer "F.Cu") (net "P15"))
 (segment (start 120.093 79.364) (end 118.875 78.146) (width 0.4) (layer "B.Cu") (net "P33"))
 (segment (start 119.058 168.122) (end 119.058 80.399) (width 0.4) (layer "B.Cu") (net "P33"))
 (segment (start 118.875 78.146) (end 118.875 53.729) (width 0.4) (layer "B.Cu") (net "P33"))
 (segment (start 119.058 80.399) (end 120.093 79.364) (width 0.4) (layer "B.Cu") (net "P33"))
 (segment (start 120.142 169.206) (end 119.058 168.122) (width 0.4) (layer "B.Cu") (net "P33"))
 (segment (start 118.875 53.729) (end 119.91 52.694) (width 0.4) (layer "B.Cu") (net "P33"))
 (segment (start 91.118 80.399) (end 92.153 79.364) (width 0.4) (layer "B.Cu") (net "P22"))
 (segment (start 92.153 79.364) (end 90.465 77.676) (width 0.4) (layer "B.Cu") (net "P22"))
 (segment (start 90.465 77.676) (end 90.465 54.199) (width 0.4) (layer "B.Cu") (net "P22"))
 (segment (start 90.465 54.199) (end 91.97 52.694) (width 0.4) (layer "B.Cu") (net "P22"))
 (segment (start 91.118 167.622) (end 91.118 80.399) (width 0.4) (layer "B.Cu") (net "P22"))
 (segment (start 92.202 168.706) (end 91.118 167.622) (width 0.4) (layer "B.Cu") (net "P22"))
 (segment (start 107.442 168.706) (end 106.358 167.622) (width 0.4) (layer "B.Cu") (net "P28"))
 (segment (start 106.175 53.729) (end 107.21 52.694) (width 0.4) (layer "B.Cu") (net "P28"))
 (segment (start 106.175 78.146) (end 106.175 53.729) (width 0.4) (layer "B.Cu") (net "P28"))
 (segment (start 106.358 80.399) (end 107.393 79.364) (width 0.4) (layer "B.Cu") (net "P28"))
 (segment (start 107.393 79.364) (end 106.175 78.146) (width 0.4) (layer "B.Cu") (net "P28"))
 (segment (start 106.358 167.622) (end 106.358 80.399) (width 0.4) (layer "B.Cu") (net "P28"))
 (segment (start 92.202 83.223) (end 92.153 83.174) (width 0.4) (layer "F.Cu") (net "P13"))
 (segment (start 92.153 83.174) (end 91.118 82.139) (width 0.4) (layer "F.Cu") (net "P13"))
 (segment (start 92.202 168.706) (end 92.202 83.223) (width 0.4) (layer "F.Cu") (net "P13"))
 (segment (start 91.118 82.139) (end 91.118 57.356) (width 0.4) (layer "F.Cu") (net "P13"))
 (segment (start 91.118 57.356) (end 91.97 56.504) (width 0.4) (layer "F.Cu") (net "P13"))
 (segment (start 108.898 82.139) (end 108.898 57.356) (width 0.4) (layer "F.Cu") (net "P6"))
 (segment (start 108.898 57.356) (end 109.75 56.504) (width 0.4) (layer "F.Cu") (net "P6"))
 (segment (start 109.982 168.706) (end 109.982 83.223) (width 0.4) (layer "F.Cu") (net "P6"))
 (segment (start 109.933 83.174) (end 108.898 82.139) (width 0.4) (layer "F.Cu") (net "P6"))
 (segment (start 116.335 78.146) (end 116.335 53.729) (width 0.4) (layer "B.Cu") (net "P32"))
 (segment (start 116.518 167.622) (end 116.518 80.399) (width 0.4) (layer "B.Cu") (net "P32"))
 (segment (start 116.335 53.729) (end 117.37 52.694) (width 0.4) (layer "B.Cu") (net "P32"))
 (segment (start 117.602 168.706) (end 116.518 167.622) (width 0.4) (layer "B.Cu") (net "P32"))
 (segment (start 116.518 80.399) (end 117.553 79.364) (width 0.4) (layer "B.Cu") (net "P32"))
 (segment (start 117.553 79.364) (end 116.335 78.146) (width 0.4) (layer "B.Cu") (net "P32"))
 (segment (start 80.958 168.122) (end 80.958 80.399) (width 0.4) (layer "B.Cu") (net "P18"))
 (segment (start 81.993 79.364) (end 80.775 78.146) (width 0.4) (layer "B.Cu") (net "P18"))
 (segment (start 80.775 53.729) (end 81.81 52.694) (width 0.4) (layer "B.Cu") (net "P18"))
 (segment (start 80.775 78.146) (end 80.775 53.729) (width 0.4) (layer "B.Cu") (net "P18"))
 (segment (start 80.958 80.399) (end 81.993 79.364) (width 0.4) (layer "B.Cu") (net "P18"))
 (segment (start 82.042 169.206) (end 80.958 168.122) (width 0.4) (layer "B.Cu") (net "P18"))
 (segment (start 102.362 168.706) (end 102.362 83.223) (width 0.4) (layer "F.Cu") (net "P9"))
 (segment (start 101.092 57.542) (end 102.13 56.504) (width 0.4) (layer "F.Cu") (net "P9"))
 (segment (start 101.092 81.953) (end 101.092 57.542) (width 0.4) (layer "F.Cu") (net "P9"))
 (segment (start 102.313 83.174) (end 101.092 81.953) (width 0.4) (layer "F.Cu") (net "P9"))
 (segment (start 108.898 167.622) (end 108.898 80.399) (width 0.4) (layer "B.Cu") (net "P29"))
 (segment (start 109.982 168.706) (end 108.898 167.622) (width 0.4) (layer "B.Cu") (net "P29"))
 (segment (start 108.898 80.399) (end 109.933 79.364) (width 0.4) (layer "B.Cu") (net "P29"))
 (segment (start 108.245 54.199) (end 109.75 52.694) (width 0.4) (layer "B.Cu") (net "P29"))
 (segment (start 108.245 77.676) (end 108.245 54.199) (width 0.4) (layer "B.Cu") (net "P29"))
 (segment (start 109.933 79.364) (end 108.245 77.676) (width 0.4) (layer "B.Cu") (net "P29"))
 (segment (start 87.073 79.364) (end 85.852 78.143) (width 0.4) (layer "B.Cu") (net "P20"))
 (segment (start 85.852 78.143) (end 85.852 53.732) (width 0.4) (layer "B.Cu") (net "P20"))
 (segment (start 85.852 53.732) (end 86.89 52.694) (width 0.4) (layer "B.Cu") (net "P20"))
 (segment (start 87.122 168.706) (end 86.038 167.622) (width 0.4) (layer "B.Cu") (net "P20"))
 (segment (start 86.038 167.622) (end 86.038 80.399) (width 0.4) (layer "B.Cu") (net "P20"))
 (segment (start 86.038 80.399) (end 87.073 79.364) (width 0.4) (layer "B.Cu") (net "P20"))
 (segment (start 104.853 83.174) (end 103.818 82.139) (width 0.4) (layer "F.Cu") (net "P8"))
 (segment (start 103.818 57.356) (end 104.67 56.504) (width 0.4) (layer "F.Cu") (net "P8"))
 (segment (start 104.902 168.706) (end 104.902 83.223) (width 0.4) (layer "F.Cu") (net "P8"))
 (segment (start 103.818 82.139) (end 103.818 57.356) (width 0.4) (layer "F.Cu") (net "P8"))
 (segment (start 117.553 83.174) (end 116.518 82.139) (width 0.4) (layer "F.Cu") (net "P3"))
 (segment (start 116.518 57.356) (end 117.37 56.504) (width 0.4) (layer "F.Cu") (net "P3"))
 (segment (start 116.518 82.139) (end 116.518 57.356) (width 0.4) (layer "F.Cu") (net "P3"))
 (segment (start 117.602 168.706) (end 117.602 83.223) (width 0.4) (layer "F.Cu") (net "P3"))
 (segment (start 97.282 168.706) (end 96.198 167.622) (width 0.4) (layer "B.Cu") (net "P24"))
 (segment (start 96.198 80.399) (end 97.233 79.364) (width 0.4) (layer "B.Cu") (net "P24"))
 (segment (start 96.015 53.729) (end 97.05 52.694) (width 0.4) (layer "B.Cu") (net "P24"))
 (segment (start 97.233 79.364) (end 96.015 78.146) (width 0.4) (layer "B.Cu") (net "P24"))
 (segment (start 96.015 78.146) (end 96.015 53.729) (width 0.4) (layer "B.Cu") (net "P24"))
 (segment (start 96.198 167.622) (end 96.198 80.399) (width 0.4) (layer "B.Cu") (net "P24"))
 (segment (start 121.598 57.356) (end 122.45 56.504) (width 0.4) (layer "F.Cu") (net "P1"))
 (segment (start 122.682 83.223) (end 122.633 83.174) (width 0.4) (layer "F.Cu") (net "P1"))
 (segment (start 122.633 83.174) (end 121.598 82.139) (width 0.4) (layer "F.Cu") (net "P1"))
 (segment (start 122.682 169.206) (end 122.682 83.223) (width 0.4) (layer "F.Cu") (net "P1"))
 (segment (start 121.598 82.139) (end 121.598 57.356) (width 0.4) (layer "F.Cu") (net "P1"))
 (segment (start 121.598 80.399) (end 122.633 79.364) (width 0.4) (layer "B.Cu") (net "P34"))
 (segment (start 122.633 79.364) (end 121.412 78.143) (width 0.4) (layer "B.Cu") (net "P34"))
 (segment (start 122.682 169.206) (end 121.598 168.122) (width 0.4) (layer "B.Cu") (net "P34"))
 (segment (start 121.412 53.732) (end 122.45 52.694) (width 0.4) (layer "B.Cu") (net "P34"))
 (segment (start 121.598 168.122) (end 121.598 80.399) (width 0.4) (layer "B.Cu") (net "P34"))
 (segment (start 121.412 78.143) (end 121.412 53.732) (width 0.4) (layer "B.Cu") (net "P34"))
 (segment (start 84.582 83.223) (end 84.533 83.174) (width 0.4) (layer "F.Cu") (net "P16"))
 (segment (start 83.498 57.356) (end 84.35 56.504) (width 0.4) (layer "F.Cu") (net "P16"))
 (segment (start 84.582 169.206) (end 84.582 83.223) (width 0.4) (layer "F.Cu") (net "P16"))
 (segment (start 83.498 82.139) (end 83.498 57.356) (width 0.4) (layer "F.Cu") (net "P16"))
 (segment (start 84.533 83.174) (end 83.498 82.139) (width 0.4) (layer "F.Cu") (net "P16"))
 (segment (start 111.438 82.139) (end 111.438 57.356) (width 0.4) (layer "F.Cu") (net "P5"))
 (segment (start 111.438 57.356) (end 112.29 56.504) (width 0.4) (layer "F.Cu") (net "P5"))
 (segment (start 112.522 168.706) (end 112.522 83.223) (width 0.4) (layer "F.Cu") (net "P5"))
 (segment (start 112.473 83.174) (end 111.438 82.139) (width 0.4) (layer "F.Cu") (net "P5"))
 (segment (start 94.742 83.223) (end 94.693 83.174) (width 0.4) (layer "F.Cu") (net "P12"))
 (segment (start 93.658 57.356) (end 94.51 56.504) (width 0.4) (layer "F.Cu") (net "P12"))
 (segment (start 94.693 83.174) (end 93.658 82.139) (width 0.4) (layer "F.Cu") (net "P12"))
 (segment (start 94.742 168.706) (end 94.742 83.223) (width 0.4) (layer "F.Cu") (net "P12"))
 (segment (start 93.658 82.139) (end 93.658 57.356) (width 0.4) (layer "F.Cu") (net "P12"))
 (segment (start 102.362 168.706) (end 101.278 167.622) (width 0.4) (layer "B.Cu") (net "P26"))
 (segment (start 101.278 80.399) (end 102.313 79.364) (width 0.4) (layer "B.Cu") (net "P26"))
 (segment (start 102.313 79.364) (end 101.095 78.146) (width 0.4) (layer "B.Cu") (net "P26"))
 (segment (start 101.278 167.622) (end 101.278 80.399) (width 0.4) (layer "B.Cu") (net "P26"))
 (segment (start 101.095 78.146) (end 101.095 53.729) (width 0.4) (layer "B.Cu") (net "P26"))
 (segment (start 101.095 53.729) (end 102.13 52.694) (width 0.4) (layer "B.Cu") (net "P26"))
 (segment (start 119.058 57.356) (end 119.91 56.504) (width 0.4) (layer "F.Cu") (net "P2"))
 (segment (start 120.093 83.174) (end 119.058 82.139) (width 0.4) (layer "F.Cu") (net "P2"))
 (segment (start 120.182 169.206) (end 120.182 83.263) (width 0.4) (layer "F.Cu") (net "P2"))
 (segment (start 119.058 82.139) (end 119.058 57.356) (width 0.4) (layer "F.Cu") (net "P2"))
 (segment (start 99.773 79.364) (end 98.555 78.146) (width 0.4) (layer "B.Cu") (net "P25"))
 (segment (start 98.555 78.146) (end 98.555 53.729) (width 0.4) (layer "B.Cu") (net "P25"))
 (segment (start 99.822 168.706) (end 98.738 167.622) (width 0.4) (layer "B.Cu") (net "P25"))
 (segment (start 98.738 80.399) (end 99.773 79.364) (width 0.4) (layer "B.Cu") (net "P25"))
 (segment (start 98.555 53.729) (end 99.59 52.694) (width 0.4) (layer "B.Cu") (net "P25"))
 (segment (start 98.738 167.622) (end 98.738 80.399) (width 0.4) (layer "B.Cu") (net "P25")))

